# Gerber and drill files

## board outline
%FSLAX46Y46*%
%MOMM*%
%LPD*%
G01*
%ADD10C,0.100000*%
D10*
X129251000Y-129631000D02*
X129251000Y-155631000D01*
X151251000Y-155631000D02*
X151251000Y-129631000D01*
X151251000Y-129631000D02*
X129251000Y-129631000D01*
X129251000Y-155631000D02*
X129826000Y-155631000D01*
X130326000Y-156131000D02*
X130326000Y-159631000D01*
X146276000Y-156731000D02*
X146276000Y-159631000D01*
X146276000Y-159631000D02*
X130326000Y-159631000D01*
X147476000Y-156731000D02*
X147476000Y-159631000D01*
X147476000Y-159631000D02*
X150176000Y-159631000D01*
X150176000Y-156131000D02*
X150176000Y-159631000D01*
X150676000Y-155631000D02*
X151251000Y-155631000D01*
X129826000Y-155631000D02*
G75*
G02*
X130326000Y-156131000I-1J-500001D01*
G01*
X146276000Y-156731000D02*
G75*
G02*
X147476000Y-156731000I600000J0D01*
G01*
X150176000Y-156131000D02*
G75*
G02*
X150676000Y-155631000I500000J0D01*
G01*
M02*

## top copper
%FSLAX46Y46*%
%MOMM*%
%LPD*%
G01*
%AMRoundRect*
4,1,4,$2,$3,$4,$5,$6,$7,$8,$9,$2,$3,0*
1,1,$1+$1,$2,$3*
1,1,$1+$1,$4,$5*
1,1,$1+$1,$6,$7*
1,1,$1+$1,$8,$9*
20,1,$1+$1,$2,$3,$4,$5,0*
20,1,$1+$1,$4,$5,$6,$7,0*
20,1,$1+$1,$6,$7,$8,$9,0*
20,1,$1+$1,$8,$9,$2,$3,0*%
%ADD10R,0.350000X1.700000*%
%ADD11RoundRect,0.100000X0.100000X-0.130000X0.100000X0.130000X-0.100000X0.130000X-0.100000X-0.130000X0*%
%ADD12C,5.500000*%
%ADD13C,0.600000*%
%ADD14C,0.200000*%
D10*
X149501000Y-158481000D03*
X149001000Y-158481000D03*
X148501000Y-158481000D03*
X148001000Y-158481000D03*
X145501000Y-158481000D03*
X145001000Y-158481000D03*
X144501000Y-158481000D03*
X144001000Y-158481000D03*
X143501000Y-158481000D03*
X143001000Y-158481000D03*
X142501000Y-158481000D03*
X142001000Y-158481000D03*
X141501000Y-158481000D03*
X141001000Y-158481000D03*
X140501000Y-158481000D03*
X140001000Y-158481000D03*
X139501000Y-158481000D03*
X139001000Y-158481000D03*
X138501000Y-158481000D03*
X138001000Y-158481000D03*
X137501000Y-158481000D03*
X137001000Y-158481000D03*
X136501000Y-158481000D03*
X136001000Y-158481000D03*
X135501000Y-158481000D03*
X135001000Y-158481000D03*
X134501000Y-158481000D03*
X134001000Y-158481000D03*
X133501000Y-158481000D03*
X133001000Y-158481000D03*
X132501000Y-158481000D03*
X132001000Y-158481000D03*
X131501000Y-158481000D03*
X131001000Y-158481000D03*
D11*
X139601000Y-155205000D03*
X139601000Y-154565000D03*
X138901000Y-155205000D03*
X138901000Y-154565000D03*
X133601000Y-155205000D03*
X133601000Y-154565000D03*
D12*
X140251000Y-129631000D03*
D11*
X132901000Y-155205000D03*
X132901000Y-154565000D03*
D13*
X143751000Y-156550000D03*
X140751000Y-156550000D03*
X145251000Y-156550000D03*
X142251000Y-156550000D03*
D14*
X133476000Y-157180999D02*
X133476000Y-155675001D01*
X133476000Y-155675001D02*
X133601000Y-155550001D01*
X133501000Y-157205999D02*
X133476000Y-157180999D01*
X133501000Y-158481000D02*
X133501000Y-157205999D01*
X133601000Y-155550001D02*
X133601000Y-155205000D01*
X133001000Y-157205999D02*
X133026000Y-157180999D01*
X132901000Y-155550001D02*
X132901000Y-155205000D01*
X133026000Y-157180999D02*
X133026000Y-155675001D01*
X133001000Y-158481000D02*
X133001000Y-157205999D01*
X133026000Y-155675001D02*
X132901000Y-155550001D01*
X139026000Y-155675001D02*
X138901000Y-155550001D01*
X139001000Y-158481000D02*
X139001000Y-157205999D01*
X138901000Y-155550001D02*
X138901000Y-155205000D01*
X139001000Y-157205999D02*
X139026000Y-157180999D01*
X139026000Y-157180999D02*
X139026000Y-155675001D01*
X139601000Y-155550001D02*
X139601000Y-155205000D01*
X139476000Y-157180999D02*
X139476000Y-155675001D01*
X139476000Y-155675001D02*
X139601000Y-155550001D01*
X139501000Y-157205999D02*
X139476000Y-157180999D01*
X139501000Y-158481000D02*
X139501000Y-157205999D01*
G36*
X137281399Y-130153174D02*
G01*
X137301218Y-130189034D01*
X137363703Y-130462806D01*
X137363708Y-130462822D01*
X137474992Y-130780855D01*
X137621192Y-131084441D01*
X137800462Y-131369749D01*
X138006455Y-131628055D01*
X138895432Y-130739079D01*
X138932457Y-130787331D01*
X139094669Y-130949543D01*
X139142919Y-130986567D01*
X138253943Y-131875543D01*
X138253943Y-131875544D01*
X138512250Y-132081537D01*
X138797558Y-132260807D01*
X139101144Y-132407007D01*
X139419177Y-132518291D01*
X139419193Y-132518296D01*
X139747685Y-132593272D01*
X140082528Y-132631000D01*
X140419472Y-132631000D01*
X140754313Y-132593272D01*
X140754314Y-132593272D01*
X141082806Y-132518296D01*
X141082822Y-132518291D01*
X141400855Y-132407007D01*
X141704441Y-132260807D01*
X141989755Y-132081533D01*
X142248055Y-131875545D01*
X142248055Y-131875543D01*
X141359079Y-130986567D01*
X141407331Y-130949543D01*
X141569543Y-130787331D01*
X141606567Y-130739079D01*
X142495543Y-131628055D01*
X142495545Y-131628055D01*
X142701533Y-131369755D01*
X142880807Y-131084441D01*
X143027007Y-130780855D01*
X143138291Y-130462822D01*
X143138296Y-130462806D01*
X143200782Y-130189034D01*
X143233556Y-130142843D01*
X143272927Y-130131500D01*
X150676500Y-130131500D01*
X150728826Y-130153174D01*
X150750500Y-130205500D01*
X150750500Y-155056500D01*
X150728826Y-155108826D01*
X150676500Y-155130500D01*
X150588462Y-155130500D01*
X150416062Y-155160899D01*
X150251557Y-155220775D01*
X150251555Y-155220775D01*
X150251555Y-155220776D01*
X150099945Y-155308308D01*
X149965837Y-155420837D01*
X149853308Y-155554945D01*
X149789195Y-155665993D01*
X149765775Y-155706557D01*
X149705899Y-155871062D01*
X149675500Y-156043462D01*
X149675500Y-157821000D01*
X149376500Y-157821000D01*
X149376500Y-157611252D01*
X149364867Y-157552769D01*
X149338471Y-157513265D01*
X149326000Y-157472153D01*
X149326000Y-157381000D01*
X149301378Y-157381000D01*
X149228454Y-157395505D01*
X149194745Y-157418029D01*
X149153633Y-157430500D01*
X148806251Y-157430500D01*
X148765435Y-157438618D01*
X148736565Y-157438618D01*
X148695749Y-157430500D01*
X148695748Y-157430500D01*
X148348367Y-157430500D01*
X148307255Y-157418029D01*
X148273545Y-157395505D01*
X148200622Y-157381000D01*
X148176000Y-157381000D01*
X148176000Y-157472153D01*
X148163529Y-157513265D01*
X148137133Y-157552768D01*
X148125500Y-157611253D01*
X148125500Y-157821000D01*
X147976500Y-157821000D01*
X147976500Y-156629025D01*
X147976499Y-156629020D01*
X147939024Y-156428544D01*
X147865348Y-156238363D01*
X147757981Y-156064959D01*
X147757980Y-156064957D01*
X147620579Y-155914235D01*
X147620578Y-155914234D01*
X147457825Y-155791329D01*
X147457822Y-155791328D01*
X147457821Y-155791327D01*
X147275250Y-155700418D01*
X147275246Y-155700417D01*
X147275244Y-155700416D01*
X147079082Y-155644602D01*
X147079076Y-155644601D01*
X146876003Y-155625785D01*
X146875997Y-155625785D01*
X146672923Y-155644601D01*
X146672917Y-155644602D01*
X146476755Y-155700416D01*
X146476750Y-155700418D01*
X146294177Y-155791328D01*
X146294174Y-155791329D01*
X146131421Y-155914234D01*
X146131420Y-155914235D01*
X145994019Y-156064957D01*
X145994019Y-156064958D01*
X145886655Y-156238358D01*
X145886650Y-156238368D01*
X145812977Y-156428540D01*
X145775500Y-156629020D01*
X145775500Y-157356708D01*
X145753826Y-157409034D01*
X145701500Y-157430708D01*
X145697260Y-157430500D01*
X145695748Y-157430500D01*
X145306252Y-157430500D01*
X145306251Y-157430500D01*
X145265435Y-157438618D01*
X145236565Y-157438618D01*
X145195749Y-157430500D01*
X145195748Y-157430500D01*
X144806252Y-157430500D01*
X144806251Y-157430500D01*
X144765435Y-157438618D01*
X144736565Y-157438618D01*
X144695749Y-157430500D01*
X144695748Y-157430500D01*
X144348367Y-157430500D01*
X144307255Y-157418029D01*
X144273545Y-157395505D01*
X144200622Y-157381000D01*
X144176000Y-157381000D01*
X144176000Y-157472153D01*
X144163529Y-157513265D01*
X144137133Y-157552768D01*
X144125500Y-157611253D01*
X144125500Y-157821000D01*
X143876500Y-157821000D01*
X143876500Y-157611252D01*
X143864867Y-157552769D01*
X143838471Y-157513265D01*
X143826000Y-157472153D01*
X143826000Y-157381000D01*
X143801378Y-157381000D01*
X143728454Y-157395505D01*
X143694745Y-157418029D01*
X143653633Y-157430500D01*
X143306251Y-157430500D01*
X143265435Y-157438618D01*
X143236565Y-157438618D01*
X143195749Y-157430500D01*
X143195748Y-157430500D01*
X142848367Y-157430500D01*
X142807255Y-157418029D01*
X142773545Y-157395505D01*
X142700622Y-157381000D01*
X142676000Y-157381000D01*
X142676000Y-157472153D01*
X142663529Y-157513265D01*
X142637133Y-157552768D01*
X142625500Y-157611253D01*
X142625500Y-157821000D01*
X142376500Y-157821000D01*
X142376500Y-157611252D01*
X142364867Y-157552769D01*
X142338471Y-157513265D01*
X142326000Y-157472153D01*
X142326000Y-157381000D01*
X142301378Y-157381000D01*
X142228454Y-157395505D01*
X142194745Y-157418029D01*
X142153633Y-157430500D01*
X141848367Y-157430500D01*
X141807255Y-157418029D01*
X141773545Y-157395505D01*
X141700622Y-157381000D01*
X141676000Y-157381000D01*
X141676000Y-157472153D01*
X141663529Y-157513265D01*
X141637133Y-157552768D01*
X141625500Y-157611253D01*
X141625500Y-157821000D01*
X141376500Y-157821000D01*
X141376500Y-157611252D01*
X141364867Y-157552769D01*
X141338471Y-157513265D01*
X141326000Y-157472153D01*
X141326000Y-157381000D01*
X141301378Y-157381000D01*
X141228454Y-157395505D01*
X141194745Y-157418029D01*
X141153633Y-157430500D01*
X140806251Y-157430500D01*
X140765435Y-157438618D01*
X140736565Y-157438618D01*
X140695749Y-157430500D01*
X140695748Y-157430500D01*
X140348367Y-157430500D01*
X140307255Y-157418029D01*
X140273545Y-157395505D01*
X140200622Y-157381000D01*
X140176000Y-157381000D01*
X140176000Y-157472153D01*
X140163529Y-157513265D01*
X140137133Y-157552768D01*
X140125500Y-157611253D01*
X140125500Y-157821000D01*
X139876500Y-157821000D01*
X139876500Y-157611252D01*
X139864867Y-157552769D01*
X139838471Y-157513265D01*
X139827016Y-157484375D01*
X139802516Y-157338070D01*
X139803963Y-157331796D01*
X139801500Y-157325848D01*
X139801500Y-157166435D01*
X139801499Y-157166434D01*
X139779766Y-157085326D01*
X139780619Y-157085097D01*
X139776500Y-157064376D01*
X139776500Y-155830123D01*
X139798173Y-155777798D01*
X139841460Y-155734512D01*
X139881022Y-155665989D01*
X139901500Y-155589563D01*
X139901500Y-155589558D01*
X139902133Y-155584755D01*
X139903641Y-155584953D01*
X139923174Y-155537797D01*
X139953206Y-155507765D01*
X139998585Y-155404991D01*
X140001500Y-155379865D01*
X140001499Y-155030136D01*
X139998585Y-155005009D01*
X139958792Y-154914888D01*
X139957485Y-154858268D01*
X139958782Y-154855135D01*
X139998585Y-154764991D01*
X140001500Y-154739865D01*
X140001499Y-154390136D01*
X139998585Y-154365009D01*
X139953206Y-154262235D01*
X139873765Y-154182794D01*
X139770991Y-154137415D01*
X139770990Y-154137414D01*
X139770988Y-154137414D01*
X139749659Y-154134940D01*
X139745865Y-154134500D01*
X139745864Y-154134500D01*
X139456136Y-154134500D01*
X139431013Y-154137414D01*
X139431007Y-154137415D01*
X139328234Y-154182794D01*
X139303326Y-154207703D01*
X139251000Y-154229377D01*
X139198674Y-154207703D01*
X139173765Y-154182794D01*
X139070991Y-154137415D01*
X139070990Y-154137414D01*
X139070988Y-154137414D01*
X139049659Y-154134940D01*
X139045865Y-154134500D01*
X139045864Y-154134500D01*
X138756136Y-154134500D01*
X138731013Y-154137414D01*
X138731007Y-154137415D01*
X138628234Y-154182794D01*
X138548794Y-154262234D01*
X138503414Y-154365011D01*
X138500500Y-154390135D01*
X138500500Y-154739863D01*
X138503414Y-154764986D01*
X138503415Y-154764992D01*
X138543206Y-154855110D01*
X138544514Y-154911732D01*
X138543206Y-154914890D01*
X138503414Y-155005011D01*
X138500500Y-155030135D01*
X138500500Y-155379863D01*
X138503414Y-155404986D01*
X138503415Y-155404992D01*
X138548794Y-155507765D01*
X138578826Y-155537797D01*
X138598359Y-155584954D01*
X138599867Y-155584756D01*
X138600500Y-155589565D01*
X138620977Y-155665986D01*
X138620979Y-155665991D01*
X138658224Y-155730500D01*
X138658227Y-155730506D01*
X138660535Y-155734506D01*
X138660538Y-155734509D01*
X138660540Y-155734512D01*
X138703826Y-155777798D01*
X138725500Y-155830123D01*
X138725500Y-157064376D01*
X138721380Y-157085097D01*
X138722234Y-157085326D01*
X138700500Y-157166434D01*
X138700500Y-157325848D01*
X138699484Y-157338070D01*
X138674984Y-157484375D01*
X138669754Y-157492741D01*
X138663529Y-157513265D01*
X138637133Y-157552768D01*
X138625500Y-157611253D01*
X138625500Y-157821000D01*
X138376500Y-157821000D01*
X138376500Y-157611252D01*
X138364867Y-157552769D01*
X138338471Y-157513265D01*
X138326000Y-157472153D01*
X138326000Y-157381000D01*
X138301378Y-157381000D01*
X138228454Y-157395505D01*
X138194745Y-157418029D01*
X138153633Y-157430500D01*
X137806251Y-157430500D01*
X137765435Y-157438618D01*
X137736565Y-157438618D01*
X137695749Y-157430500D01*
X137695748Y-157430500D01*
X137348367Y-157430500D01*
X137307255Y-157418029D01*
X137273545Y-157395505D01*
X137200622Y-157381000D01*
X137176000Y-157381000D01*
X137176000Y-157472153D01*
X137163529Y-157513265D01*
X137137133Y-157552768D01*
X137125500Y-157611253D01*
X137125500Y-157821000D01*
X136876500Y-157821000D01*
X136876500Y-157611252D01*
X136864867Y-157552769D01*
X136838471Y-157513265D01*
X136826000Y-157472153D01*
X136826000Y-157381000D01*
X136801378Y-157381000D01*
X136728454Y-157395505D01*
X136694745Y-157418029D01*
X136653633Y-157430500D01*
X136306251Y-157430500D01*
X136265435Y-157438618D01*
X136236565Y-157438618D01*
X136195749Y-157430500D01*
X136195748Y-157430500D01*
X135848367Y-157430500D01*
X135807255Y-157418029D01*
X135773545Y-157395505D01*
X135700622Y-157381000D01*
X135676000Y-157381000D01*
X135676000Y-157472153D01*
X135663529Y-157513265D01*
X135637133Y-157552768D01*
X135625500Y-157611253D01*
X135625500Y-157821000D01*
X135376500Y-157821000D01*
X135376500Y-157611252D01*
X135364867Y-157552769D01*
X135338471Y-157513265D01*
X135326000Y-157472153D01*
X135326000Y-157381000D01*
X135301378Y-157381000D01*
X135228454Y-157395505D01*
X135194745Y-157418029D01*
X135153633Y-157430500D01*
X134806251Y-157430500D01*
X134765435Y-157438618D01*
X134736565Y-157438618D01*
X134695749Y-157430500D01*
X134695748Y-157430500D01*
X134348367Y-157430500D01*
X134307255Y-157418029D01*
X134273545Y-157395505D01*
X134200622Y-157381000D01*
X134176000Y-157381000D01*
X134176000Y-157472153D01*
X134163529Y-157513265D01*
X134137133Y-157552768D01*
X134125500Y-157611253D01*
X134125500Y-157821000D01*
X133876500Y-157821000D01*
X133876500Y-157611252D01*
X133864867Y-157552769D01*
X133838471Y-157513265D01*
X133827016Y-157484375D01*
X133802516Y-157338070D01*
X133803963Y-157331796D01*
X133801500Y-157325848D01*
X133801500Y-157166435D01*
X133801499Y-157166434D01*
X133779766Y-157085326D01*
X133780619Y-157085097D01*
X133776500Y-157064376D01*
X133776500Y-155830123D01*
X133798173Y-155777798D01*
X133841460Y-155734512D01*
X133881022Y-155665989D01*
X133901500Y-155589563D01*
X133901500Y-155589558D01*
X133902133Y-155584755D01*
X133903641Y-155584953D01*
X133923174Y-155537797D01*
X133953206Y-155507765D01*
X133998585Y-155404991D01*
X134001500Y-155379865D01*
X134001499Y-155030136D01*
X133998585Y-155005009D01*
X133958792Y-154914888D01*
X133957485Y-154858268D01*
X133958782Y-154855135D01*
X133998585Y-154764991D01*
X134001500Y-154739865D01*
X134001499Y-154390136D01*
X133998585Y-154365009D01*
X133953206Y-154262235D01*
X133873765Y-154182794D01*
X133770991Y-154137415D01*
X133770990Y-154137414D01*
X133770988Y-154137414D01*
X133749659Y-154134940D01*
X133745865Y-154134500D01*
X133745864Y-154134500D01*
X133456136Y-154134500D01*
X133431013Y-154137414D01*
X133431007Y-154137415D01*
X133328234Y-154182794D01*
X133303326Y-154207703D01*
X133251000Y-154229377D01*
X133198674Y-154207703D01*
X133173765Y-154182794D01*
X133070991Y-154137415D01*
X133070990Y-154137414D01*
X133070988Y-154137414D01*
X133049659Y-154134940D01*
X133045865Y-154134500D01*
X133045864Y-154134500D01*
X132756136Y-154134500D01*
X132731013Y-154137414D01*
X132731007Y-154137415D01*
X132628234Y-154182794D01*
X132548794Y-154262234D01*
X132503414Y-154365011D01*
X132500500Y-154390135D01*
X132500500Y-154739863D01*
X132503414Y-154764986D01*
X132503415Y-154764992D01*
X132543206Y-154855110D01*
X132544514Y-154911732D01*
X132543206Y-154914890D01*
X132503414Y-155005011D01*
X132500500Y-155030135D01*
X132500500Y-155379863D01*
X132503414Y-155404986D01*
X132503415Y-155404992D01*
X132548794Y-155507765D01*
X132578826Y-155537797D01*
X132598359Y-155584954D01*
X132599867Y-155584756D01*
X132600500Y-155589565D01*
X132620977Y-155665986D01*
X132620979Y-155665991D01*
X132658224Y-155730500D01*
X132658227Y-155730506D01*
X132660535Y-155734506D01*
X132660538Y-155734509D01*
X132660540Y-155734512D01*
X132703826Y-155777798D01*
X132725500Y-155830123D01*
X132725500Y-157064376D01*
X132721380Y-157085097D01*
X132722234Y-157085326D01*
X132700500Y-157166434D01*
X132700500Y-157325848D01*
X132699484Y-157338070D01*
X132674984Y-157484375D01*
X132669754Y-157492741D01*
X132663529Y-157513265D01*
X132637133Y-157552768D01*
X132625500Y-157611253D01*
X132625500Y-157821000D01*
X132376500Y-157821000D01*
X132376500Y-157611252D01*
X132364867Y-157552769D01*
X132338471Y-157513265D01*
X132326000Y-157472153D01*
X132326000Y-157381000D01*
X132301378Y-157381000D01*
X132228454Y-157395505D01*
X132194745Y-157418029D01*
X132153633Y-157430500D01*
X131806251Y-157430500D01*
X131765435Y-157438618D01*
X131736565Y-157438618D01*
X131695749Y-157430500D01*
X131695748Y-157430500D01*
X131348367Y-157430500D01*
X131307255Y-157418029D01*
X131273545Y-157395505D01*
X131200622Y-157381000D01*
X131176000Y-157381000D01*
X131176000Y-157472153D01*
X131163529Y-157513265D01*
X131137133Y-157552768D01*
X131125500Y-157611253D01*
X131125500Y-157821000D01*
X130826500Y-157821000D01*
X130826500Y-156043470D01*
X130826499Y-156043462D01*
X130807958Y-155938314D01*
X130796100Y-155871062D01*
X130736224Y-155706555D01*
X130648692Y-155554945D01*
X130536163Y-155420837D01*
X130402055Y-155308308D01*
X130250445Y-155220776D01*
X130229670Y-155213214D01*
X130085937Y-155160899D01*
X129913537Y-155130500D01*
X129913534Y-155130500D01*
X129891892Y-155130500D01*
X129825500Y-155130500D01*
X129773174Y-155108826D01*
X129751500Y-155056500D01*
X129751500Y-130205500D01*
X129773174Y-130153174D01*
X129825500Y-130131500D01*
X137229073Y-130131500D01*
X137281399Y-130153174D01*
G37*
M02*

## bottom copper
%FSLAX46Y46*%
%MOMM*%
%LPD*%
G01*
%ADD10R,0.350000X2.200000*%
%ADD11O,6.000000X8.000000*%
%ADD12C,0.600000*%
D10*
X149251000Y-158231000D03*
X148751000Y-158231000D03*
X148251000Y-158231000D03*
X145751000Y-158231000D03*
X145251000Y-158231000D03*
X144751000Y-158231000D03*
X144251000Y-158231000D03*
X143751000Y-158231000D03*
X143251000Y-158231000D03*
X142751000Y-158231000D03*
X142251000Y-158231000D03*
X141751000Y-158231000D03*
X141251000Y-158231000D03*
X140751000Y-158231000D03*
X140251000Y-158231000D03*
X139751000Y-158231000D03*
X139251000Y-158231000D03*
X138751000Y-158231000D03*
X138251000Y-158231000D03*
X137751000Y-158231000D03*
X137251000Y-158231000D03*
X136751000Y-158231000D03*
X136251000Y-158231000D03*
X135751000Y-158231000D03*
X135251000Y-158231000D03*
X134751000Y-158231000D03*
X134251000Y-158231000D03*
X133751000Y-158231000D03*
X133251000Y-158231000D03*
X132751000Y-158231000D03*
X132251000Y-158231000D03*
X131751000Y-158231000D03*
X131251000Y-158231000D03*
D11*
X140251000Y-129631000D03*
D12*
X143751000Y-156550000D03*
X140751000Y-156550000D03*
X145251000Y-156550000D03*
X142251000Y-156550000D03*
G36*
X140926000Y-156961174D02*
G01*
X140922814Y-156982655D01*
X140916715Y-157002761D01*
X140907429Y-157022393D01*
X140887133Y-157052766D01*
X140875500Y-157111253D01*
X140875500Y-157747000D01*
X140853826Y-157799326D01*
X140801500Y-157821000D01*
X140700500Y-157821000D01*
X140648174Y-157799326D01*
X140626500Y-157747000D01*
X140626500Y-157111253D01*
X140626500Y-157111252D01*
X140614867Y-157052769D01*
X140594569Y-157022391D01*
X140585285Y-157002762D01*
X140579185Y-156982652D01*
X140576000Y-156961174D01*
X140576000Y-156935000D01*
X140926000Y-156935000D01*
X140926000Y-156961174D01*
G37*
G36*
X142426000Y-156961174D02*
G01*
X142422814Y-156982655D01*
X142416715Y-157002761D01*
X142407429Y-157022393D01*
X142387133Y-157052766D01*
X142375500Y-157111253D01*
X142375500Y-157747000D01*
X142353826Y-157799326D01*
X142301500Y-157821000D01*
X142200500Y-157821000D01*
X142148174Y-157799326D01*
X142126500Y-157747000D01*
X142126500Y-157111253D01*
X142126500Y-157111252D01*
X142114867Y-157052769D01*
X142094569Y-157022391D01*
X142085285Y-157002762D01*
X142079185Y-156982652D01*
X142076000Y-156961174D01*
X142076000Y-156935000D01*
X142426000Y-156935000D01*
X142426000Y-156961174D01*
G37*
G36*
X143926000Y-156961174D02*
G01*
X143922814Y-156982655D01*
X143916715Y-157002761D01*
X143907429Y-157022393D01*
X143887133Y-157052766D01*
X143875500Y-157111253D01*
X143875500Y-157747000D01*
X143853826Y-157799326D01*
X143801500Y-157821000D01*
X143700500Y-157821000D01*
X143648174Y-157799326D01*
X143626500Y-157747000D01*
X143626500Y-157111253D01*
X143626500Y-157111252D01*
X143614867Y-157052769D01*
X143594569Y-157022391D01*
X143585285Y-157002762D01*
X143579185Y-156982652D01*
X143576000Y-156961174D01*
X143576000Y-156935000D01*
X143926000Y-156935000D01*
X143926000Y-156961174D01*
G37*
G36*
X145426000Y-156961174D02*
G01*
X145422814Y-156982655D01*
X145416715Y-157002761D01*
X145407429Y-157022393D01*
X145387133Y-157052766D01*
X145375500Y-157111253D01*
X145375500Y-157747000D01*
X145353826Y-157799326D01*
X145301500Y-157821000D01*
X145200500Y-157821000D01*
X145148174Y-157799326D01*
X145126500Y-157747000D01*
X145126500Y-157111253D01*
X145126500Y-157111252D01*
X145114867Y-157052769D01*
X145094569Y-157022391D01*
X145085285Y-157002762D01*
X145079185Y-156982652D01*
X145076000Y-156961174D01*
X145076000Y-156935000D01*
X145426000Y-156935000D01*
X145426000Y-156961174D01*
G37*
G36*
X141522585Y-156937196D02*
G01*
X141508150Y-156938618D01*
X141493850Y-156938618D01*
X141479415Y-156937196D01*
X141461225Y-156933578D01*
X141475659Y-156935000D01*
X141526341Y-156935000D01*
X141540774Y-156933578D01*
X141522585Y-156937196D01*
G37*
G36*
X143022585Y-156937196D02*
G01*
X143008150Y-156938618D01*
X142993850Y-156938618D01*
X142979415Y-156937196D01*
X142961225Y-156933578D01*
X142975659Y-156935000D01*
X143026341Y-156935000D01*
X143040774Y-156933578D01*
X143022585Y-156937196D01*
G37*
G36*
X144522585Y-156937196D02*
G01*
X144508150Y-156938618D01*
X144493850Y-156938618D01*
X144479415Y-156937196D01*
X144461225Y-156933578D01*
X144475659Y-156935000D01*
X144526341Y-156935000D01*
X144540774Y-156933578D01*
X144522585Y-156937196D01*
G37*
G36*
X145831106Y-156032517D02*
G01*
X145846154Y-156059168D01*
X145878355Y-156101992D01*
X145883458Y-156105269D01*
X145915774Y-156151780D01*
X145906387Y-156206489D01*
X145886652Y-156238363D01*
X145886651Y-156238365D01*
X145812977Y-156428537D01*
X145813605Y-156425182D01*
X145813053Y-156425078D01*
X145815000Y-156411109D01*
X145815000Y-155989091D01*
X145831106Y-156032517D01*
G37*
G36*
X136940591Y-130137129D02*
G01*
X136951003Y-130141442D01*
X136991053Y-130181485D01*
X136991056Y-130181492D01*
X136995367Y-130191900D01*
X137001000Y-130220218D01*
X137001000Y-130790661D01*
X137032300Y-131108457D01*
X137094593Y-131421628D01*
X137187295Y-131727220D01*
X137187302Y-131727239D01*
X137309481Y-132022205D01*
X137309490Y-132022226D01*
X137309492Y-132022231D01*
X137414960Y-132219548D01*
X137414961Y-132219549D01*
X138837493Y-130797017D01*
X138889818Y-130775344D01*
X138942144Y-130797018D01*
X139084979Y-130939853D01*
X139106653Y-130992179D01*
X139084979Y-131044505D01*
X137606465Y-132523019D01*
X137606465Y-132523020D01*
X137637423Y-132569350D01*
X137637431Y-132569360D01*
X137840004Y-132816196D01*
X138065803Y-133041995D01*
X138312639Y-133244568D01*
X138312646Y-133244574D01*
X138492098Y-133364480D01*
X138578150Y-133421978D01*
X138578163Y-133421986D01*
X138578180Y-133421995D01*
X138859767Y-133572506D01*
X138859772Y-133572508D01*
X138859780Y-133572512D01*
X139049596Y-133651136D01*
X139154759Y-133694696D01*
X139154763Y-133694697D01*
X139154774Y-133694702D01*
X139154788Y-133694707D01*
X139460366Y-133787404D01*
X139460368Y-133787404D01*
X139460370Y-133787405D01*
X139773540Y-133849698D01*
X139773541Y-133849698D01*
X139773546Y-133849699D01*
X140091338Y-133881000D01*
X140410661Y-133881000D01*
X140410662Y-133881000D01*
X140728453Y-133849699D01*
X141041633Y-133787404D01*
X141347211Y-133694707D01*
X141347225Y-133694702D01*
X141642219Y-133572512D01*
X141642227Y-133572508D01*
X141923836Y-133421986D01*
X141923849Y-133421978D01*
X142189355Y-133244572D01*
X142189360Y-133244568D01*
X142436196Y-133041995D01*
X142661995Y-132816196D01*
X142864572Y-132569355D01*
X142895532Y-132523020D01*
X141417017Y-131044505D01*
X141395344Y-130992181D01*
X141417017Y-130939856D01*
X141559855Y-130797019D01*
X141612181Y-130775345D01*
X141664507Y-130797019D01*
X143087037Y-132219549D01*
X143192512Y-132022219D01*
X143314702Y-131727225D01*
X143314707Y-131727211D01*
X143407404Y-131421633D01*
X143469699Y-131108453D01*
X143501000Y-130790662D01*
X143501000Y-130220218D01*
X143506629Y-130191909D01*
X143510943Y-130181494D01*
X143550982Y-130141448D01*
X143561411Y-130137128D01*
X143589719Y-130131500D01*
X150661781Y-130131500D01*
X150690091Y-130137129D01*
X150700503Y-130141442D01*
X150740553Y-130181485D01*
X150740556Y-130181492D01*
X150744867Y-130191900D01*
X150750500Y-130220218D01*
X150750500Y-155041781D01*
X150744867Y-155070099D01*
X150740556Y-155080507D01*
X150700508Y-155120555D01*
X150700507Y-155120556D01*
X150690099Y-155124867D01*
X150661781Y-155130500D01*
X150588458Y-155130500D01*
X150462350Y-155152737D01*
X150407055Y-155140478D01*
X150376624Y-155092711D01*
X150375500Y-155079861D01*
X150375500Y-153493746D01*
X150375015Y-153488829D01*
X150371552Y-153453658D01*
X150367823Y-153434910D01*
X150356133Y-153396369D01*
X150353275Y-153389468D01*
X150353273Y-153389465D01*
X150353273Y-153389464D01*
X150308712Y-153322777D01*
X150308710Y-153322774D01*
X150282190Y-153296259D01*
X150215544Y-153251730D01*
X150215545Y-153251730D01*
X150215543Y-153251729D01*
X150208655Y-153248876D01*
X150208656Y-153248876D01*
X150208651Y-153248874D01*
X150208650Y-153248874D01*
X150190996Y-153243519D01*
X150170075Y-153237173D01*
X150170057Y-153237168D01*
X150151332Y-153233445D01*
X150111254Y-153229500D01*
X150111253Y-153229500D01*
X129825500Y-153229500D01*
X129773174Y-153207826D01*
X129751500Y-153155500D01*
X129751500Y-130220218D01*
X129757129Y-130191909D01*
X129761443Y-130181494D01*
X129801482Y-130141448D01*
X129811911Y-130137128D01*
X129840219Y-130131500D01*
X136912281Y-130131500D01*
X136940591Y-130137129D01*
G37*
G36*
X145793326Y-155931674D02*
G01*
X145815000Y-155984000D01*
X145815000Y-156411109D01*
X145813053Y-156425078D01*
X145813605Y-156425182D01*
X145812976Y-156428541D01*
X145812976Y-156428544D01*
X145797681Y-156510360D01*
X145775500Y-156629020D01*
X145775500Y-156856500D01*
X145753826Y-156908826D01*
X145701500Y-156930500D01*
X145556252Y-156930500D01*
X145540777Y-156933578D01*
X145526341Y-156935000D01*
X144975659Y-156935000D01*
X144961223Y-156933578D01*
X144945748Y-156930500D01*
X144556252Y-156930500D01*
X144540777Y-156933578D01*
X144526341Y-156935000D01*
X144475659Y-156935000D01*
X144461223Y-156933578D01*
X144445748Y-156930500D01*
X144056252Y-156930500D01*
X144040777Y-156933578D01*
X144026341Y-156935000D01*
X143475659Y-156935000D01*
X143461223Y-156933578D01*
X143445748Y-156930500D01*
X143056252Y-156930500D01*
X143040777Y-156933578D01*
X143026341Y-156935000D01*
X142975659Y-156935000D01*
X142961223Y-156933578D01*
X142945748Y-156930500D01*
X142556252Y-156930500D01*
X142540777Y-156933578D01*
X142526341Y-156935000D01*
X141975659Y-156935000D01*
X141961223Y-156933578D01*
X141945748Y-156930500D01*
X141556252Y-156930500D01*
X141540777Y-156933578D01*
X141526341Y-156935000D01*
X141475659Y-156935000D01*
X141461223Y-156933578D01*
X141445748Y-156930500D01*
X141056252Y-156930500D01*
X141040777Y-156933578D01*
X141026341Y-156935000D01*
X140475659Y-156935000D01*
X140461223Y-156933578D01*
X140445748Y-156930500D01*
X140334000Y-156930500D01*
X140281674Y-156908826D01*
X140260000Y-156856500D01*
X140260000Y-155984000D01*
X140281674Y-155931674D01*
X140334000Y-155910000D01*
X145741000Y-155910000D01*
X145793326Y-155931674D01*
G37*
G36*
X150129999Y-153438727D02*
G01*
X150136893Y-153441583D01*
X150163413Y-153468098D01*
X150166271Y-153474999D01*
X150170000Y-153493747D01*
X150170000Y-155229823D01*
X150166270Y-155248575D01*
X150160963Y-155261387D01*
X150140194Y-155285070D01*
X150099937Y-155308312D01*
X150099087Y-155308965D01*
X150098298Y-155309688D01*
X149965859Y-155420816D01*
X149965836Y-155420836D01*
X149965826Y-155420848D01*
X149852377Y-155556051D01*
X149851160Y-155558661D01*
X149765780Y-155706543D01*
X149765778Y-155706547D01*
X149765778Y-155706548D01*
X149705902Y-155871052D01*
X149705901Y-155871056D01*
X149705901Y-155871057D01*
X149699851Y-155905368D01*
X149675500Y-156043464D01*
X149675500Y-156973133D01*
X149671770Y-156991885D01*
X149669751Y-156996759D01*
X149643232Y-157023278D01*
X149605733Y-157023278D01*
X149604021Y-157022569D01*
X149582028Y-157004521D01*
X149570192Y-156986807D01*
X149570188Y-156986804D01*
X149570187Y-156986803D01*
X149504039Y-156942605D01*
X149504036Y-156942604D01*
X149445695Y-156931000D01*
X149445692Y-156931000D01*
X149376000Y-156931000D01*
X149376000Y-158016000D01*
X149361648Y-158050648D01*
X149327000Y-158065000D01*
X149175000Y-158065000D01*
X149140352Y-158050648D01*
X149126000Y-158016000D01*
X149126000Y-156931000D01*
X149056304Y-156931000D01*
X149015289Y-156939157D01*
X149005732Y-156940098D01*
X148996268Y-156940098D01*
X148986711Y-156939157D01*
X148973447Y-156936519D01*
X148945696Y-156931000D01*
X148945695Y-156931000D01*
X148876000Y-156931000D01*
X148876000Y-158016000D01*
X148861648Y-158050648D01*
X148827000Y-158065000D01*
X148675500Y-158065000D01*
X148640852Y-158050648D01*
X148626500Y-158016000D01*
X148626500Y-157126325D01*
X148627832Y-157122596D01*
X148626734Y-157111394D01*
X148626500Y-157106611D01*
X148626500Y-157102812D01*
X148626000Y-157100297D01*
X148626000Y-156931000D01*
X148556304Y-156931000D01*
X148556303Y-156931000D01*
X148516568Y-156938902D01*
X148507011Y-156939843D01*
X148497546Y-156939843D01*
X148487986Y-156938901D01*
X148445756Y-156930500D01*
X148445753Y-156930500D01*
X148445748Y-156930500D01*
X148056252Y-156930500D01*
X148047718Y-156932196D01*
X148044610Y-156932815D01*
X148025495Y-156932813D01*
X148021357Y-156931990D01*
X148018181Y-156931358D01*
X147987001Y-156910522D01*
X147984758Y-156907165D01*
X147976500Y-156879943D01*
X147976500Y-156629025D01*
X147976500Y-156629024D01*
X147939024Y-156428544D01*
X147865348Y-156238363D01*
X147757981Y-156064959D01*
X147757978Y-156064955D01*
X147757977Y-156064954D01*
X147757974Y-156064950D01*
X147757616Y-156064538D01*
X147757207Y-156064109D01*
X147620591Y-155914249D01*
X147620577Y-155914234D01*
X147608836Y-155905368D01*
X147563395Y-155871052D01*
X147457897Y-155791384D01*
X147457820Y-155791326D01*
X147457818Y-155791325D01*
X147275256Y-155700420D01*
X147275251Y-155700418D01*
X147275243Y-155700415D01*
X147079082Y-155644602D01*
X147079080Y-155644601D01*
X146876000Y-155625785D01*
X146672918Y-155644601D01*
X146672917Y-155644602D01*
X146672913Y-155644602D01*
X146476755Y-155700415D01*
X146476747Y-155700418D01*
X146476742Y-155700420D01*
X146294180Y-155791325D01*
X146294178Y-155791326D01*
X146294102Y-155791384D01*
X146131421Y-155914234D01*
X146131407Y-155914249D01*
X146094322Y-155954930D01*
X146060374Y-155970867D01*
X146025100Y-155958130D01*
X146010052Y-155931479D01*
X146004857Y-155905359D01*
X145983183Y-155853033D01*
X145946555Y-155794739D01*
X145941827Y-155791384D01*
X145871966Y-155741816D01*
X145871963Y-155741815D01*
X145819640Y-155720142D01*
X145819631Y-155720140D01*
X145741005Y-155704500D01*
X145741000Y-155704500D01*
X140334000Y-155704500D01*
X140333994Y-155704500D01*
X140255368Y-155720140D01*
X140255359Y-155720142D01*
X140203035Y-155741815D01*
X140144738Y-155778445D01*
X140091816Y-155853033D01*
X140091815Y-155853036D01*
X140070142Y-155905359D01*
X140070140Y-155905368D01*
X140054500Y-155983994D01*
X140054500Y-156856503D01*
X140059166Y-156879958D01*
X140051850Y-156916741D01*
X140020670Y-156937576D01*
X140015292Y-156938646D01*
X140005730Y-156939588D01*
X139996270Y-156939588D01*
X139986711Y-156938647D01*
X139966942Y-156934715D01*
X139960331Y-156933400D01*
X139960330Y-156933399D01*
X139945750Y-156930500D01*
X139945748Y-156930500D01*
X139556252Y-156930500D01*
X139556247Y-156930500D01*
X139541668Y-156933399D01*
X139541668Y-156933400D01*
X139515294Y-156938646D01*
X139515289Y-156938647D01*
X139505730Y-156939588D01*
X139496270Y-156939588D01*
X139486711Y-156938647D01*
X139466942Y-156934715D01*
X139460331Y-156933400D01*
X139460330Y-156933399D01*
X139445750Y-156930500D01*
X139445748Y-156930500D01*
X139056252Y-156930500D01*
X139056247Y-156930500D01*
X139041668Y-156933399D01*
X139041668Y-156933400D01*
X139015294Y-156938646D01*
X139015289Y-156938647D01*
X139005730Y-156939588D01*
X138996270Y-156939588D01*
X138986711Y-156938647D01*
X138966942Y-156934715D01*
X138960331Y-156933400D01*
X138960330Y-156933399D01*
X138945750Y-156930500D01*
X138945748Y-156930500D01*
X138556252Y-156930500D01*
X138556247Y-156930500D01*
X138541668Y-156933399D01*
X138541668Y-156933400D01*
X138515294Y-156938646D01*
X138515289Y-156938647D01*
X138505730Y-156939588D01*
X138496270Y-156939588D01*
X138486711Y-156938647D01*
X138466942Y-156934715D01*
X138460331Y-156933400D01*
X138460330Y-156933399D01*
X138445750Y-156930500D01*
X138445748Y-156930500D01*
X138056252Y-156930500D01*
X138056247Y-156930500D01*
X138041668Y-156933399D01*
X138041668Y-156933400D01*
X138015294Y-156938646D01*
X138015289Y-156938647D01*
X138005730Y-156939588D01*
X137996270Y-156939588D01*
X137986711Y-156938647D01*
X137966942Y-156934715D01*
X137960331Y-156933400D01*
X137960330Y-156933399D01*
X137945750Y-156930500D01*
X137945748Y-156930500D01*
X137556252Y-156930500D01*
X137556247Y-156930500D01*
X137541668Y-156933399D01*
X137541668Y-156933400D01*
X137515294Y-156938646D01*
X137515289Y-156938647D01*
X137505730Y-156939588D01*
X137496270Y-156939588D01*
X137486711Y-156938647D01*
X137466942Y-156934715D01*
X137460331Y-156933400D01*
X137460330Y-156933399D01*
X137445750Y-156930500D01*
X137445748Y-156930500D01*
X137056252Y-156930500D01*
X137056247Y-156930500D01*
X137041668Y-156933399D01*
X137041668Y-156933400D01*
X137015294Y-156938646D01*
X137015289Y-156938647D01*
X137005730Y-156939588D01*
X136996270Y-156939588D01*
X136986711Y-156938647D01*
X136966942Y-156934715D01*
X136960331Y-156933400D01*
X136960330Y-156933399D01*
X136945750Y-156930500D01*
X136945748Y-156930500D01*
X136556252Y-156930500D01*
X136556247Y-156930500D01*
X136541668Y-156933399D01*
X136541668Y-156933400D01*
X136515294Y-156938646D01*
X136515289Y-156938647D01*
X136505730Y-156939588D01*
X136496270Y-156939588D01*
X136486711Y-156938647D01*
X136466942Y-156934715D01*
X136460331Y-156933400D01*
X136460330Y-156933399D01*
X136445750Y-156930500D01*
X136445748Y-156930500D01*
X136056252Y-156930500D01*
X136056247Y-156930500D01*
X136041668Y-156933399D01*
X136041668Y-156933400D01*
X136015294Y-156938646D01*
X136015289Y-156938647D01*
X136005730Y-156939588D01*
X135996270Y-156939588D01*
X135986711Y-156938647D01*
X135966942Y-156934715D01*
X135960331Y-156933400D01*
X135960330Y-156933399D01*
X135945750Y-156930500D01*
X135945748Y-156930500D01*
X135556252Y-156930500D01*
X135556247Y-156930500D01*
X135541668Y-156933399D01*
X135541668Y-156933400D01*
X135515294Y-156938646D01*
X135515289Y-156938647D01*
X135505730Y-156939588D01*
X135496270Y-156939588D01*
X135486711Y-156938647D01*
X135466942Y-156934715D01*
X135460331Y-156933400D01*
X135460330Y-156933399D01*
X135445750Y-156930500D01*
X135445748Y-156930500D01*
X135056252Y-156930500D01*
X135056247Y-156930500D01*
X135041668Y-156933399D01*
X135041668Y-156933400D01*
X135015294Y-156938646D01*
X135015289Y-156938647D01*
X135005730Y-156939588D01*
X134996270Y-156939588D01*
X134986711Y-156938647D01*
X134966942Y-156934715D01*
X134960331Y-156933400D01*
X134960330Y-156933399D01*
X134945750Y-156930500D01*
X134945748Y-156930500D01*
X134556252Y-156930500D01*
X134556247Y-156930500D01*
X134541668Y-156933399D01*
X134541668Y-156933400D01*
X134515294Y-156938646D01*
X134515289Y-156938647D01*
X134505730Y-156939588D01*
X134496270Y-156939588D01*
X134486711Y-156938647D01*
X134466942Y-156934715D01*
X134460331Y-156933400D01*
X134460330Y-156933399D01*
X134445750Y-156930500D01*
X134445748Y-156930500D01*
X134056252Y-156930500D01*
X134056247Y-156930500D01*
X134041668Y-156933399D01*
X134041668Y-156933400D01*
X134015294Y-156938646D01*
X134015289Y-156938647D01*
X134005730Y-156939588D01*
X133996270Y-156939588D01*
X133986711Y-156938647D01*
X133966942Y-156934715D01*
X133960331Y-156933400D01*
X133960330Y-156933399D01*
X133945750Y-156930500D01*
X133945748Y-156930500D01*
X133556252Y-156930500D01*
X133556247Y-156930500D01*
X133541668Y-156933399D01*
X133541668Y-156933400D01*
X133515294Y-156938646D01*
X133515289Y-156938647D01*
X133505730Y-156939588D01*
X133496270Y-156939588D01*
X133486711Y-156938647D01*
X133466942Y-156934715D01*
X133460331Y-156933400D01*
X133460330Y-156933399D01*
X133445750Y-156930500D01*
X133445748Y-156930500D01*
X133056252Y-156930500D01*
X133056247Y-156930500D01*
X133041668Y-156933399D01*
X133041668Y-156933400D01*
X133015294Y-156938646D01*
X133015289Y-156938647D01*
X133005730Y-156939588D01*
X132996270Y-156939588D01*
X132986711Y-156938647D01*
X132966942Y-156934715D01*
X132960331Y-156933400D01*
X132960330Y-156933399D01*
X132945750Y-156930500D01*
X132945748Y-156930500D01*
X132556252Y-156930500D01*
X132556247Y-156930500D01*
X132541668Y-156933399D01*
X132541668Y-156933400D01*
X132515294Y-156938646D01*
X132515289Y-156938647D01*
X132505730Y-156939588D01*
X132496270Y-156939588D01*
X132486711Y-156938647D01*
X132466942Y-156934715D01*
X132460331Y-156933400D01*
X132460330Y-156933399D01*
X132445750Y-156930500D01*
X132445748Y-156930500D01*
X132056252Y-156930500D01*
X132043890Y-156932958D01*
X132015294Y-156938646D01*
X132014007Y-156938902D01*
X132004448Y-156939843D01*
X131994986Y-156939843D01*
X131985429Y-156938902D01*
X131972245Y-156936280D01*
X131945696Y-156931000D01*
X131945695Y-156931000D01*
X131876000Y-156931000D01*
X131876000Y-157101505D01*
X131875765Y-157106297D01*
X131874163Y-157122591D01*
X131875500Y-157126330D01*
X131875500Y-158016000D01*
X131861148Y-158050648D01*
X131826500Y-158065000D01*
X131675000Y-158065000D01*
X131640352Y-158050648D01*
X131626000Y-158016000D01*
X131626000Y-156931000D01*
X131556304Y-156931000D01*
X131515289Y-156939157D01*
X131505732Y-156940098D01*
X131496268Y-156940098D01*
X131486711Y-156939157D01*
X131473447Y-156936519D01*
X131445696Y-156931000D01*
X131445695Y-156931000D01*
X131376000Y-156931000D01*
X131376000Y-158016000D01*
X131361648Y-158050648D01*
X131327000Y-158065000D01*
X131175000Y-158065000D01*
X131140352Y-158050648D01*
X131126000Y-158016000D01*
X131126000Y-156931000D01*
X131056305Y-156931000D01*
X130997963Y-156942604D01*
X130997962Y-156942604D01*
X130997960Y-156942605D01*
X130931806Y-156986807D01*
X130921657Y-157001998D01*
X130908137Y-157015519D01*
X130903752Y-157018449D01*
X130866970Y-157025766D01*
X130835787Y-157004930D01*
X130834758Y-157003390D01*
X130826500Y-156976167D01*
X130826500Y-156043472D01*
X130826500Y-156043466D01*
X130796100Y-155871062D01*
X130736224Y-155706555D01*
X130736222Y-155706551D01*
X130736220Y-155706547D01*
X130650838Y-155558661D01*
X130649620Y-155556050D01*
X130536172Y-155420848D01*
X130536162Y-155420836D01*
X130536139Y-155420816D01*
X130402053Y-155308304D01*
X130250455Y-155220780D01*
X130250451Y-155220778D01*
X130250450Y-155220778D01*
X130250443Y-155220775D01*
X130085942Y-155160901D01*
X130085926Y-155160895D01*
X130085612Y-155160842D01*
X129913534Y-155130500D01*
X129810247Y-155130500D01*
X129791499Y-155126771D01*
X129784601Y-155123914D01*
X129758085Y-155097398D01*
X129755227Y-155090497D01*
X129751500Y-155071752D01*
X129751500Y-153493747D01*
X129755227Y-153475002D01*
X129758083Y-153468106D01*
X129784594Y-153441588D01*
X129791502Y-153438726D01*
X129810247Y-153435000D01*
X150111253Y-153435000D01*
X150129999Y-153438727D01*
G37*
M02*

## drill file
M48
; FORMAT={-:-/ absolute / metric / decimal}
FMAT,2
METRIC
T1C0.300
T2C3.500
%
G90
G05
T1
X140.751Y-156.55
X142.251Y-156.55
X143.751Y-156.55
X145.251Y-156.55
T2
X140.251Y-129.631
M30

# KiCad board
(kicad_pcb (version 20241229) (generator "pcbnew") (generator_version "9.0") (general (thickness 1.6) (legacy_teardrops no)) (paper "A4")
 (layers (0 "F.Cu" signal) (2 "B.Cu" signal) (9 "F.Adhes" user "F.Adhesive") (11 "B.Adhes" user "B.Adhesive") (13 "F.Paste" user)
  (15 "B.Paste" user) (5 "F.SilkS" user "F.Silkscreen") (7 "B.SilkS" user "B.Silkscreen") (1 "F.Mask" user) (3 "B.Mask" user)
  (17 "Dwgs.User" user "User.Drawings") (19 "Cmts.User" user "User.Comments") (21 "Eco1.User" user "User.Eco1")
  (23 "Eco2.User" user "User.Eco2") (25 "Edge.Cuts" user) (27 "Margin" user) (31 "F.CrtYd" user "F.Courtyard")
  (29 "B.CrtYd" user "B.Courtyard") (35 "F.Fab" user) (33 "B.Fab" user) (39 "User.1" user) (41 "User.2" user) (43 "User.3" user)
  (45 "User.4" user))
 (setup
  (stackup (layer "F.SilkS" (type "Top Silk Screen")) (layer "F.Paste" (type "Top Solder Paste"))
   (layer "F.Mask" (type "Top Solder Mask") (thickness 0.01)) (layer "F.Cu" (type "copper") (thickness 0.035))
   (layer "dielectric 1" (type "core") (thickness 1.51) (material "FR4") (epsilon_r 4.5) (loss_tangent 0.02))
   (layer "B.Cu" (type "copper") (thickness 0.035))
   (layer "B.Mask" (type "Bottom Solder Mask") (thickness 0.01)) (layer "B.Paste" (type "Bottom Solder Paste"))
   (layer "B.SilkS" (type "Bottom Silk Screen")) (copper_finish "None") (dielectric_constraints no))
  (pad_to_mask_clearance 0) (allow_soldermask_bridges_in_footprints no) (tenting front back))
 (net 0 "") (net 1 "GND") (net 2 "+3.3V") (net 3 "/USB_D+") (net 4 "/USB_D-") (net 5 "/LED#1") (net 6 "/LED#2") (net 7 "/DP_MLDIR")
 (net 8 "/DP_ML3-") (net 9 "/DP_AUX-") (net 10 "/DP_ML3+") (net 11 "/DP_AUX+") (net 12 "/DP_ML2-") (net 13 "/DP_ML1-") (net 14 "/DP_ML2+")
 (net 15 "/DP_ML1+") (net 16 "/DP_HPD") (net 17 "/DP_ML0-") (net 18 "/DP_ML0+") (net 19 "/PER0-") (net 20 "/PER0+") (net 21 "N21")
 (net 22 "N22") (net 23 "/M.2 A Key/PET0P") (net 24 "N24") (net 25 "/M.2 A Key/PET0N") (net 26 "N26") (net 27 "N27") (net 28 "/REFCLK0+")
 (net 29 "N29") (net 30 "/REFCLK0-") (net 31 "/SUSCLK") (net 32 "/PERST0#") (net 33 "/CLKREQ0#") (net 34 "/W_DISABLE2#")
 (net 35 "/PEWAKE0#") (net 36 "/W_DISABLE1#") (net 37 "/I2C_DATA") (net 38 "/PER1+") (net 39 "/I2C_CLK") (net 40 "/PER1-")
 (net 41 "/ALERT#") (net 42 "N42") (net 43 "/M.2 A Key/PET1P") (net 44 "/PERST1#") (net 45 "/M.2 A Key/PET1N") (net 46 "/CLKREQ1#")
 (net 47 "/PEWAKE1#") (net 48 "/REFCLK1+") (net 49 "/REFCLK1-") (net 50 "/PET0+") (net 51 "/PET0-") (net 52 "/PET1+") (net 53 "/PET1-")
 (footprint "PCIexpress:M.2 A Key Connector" (layer "F.Cu") (at 140.251 158.521)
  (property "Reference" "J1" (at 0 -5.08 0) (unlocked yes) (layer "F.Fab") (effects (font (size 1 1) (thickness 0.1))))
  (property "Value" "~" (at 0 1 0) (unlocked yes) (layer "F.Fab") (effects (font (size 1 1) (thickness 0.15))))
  (fp_line (start -11 -2.89) (end -10.425 -2.89) (stroke (width 0.1) (type default)) (layer "Edge.Cuts"))
  (fp_line (start -9.925 -2.39) (end -9.925 1.11) (stroke (width 0.1) (type default)) (layer "Edge.Cuts"))
  (fp_line (start 6.025 -1.79) (end 6.025 1.11) (stroke (width 0.1) (type default)) (layer "Edge.Cuts"))
  (fp_line (start 6.025 1.11) (end -9.925 1.11) (stroke (width 0.1) (type default)) (layer "Edge.Cuts"))
  (fp_line (start 7.225 -1.79) (end 7.225 1.11) (stroke (width 0.1) (type default)) (layer "Edge.Cuts"))
  (fp_line (start 7.225 1.11) (end 9.925 1.11) (stroke (width 0.1) (type default)) (layer "Edge.Cuts"))
  (fp_line (start 9.925 -2.39) (end 9.925 1.11) (stroke (width 0.1) (type default)) (layer "Edge.Cuts"))
  (fp_line (start 10.425 -2.89) (end 11 -2.89) (stroke (width 0.1) (type default)) (layer "Edge.Cuts"))
  (fp_arc (start -10.425 -2.89) (mid -10.071447 -2.743553) (end -9.925 -2.39) (stroke (width 0.1) (type default)) (layer "Edge.Cuts"))
  (fp_arc (start 6.025 -1.79) (mid 6.625 -2.39) (end 7.225 -1.79) (stroke (width 0.1) (type default)) (layer "Edge.Cuts"))
  (fp_arc (start 9.925 -2.39) (mid 10.071447 -2.743553) (end 10.425 -2.89) (stroke (width 0.1) (type default)) (layer "Edge.Cuts"))
  (pad "1" smd rect (at 9.25 -0.04 180) (size 0.35 1.7) (layers "F.Cu") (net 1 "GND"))
  (pad "2" smd rect (at 9 -0.29 180) (size 0.35 2.2) (layers "B.Cu") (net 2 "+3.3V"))
  (pad "3" smd rect (at 8.75 -0.04 180) (size 0.35 1.7) (layers "F.Cu") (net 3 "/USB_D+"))
  (pad "4" smd rect (at 8.5 -0.29 180) (size 0.35 2.2) (layers "B.Cu") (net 2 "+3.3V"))
  (pad "5" smd rect (at 8.25 -0.04 180) (size 0.35 1.7) (layers "F.Cu") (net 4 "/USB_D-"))
  (pad "6" smd rect (at 8 -0.29 180) (size 0.35 2.2) (layers "B.Cu") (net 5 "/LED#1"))
  (pad "7" smd rect (at 7.75 -0.04 180) (size 0.35 1.7) (layers "F.Cu") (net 1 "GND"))
  (pad "16" smd rect (at 5.5 -0.29 180) (size 0.35 2.2) (layers "B.Cu") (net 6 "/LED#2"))
  (pad "17" smd rect (at 5.25 -0.04 180) (size 0.35 1.7) (layers "F.Cu") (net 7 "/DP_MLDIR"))
  (pad "18" smd rect (at 5 -0.29 180) (size 0.35 2.2) (layers "B.Cu") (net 1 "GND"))
  (pad "19" smd rect (at 4.75 -0.04 180) (size 0.35 1.7) (layers "F.Cu") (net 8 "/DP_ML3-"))
  (pad "20" smd rect (at 4.5 -0.29 180) (size 0.35 2.2) (layers "B.Cu") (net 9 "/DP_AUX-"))
  (pad "21" smd rect (at 4.25 -0.04 180) (size 0.35 1.7) (layers "F.Cu") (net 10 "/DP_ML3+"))
  (pad "22" smd rect (at 4 -0.29 180) (size 0.35 2.2) (layers "B.Cu") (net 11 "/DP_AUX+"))
  (pad "23" smd rect (at 3.75 -0.04 180) (size 0.35 1.7) (layers "F.Cu") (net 1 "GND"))
  (pad "24" smd rect (at 3.5 -0.29 180) (size 0.35 2.2) (layers "B.Cu") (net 1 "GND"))
  (pad "25" smd rect (at 3.25 -0.04 180) (size 0.35 1.7) (layers "F.Cu") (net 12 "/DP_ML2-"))
  (pad "26" smd rect (at 3 -0.29 180) (size 0.35 2.2) (layers "B.Cu") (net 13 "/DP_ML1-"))
  (pad "27" smd rect (at 2.75 -0.04 180) (size 0.35 1.7) (layers "F.Cu") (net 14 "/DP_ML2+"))
  (pad "28" smd rect (at 2.5 -0.29 180) (size 0.35 2.2) (layers "B.Cu") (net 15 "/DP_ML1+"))
  (pad "29" smd rect (at 2.25 -0.04 180) (size 0.35 1.7) (layers "F.Cu") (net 1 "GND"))
  (pad "30" smd rect (at 2 -0.29 180) (size 0.35 2.2) (layers "B.Cu") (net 1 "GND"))
  (pad "31" smd rect (at 1.75 -0.04 180) (size 0.35 1.7) (layers "F.Cu") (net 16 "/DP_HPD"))
  (pad "32" smd rect (at 1.5 -0.29 180) (size 0.35 2.2) (layers "B.Cu") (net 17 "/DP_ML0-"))
  (pad "33" smd rect (at 1.25 -0.04 180) (size 0.35 1.7) (layers "F.Cu") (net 1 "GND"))
  (pad "34" smd rect (at 1 -0.29 180) (size 0.35 2.2) (layers "B.Cu") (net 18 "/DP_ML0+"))
  (pad "35" smd rect (at 0.75 -0.04 180) (size 0.35 1.7) (layers "F.Cu") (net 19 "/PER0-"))
  (pad "36" smd rect (at 0.5 -0.29 180) (size 0.35 2.2) (layers "B.Cu") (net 1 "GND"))
  (pad "37" smd rect (at 0.25 -0.04 180) (size 0.35 1.7) (layers "F.Cu") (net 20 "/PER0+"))
  (pad "38" smd rect (at 0 -0.29 180) (size 0.35 2.2) (layers "B.Cu") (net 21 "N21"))
  (pad "39" smd rect (at -0.25 -0.04 180) (size 0.35 1.7) (layers "F.Cu") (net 1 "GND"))
  (pad "40" smd rect (at -0.5 -0.29 180) (size 0.35 2.2) (layers "B.Cu") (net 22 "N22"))
  (pad "41" smd rect (at -0.75 -0.04 180) (size 0.35 1.7) (layers "F.Cu") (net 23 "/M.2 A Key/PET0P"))
  (pad "42" smd rect (at -1 -0.29 180) (size 0.35 2.2) (layers "B.Cu") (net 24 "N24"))
  (pad "43" smd rect (at -1.25 -0.04 180) (size 0.35 1.7) (layers "F.Cu") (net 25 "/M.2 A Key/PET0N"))
  (pad "44" smd rect (at -1.5 -0.29 180) (size 0.35 2.2) (layers "B.Cu") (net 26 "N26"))
  (pad "45" smd rect (at -1.75 -0.04 180) (size 0.35 1.7) (layers "F.Cu") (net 1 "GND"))
  (pad "46" smd rect (at -2 -0.29 180) (size 0.35 2.2) (layers "B.Cu") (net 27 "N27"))
  (pad "47" smd rect (at -2.25 -0.04 180) (size 0.35 1.7) (layers "F.Cu") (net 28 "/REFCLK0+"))
  (pad "48" smd rect (at -2.5 -0.29 180) (size 0.35 2.2) (layers "B.Cu") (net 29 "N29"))
  (pad "49" smd rect (at -2.75 -0.04 180) (size 0.35 1.7) (layers "F.Cu") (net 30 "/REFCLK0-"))
  (pad "50" smd rect (at -3 -0.29 180) (size 0.35 2.2) (layers "B.Cu") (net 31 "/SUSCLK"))
  (pad "51" smd rect (at -3.25 -0.04 180) (size 0.35 1.7) (layers "F.Cu") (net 1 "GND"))
  (pad "52" smd rect (at -3.5 -0.29 180) (size 0.35 2.2) (layers "B.Cu") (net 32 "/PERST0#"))
  (pad "53" smd rect (at -3.75 -0.04 180) (size 0.35 1.7) (layers "F.Cu") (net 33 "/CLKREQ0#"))
  (pad "54" smd rect (at -4 -0.29 180) (size 0.35 2.2) (layers "B.Cu") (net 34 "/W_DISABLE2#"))
  (pad "55" smd rect (at -4.25 -0.04 180) (size 0.35 1.7) (layers "F.Cu") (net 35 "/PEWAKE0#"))
  (pad "56" smd rect (at -4.5 -0.29 180) (size 0.35 2.2) (layers "B.Cu") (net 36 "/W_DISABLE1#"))
  (pad "57" smd rect (at -4.75 -0.04 180) (size 0.35 1.7) (layers "F.Cu") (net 1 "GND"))
  (pad "58" smd rect (at -5 -0.29 180) (size 0.35 2.2) (layers "B.Cu") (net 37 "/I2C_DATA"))
  (pad "59" smd rect (at -5.25 -0.04 180) (size 0.35 1.7) (layers "F.Cu") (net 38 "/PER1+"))
  (pad "60" smd rect (at -5.5 -0.29 180) (size 0.35 2.2) (layers "B.Cu") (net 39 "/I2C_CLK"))
  (pad "61" smd rect (at -5.75 -0.04 180) (size 0.35 1.7) (layers "F.Cu") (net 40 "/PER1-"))
  (pad "62" smd rect (at -6 -0.29 180) (size 0.35 2.2) (layers "B.Cu") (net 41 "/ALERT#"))
  (pad "63" smd rect (at -6.25 -0.04 180) (size 0.35 1.7) (layers "F.Cu") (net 1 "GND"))
  (pad "64" smd rect (at -6.5 -0.29 180) (size 0.35 2.2) (layers "B.Cu") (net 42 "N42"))
  (pad "65" smd rect (at -6.75 -0.04 180) (size 0.35 1.7) (layers "F.Cu") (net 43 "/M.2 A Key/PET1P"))
  (pad "66" smd rect (at -7 -0.29 180) (size 0.35 2.2) (layers "B.Cu") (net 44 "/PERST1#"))
  (pad "67" smd rect (at -7.25 -0.04 180) (size 0.35 1.7) (layers "F.Cu") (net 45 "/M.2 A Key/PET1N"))
  (pad "68" smd rect (at -7.5 -0.29 180) (size 0.35 2.2) (layers "B.Cu") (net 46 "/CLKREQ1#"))
  (pad "69" smd rect (at -7.75 -0.04 180) (size 0.35 1.7) (layers "F.Cu") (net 1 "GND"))
  (pad "70" smd rect (at -8 -0.29 180) (size 0.35 2.2) (layers "B.Cu") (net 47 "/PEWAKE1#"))
  (pad "71" smd rect (at -8.25 -0.04 180) (size 0.35 1.7) (layers "F.Cu") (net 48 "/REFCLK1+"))
  (pad "72" smd rect (at -8.5 -0.29 180) (size 0.35 2.2) (layers "B.Cu") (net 2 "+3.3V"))
  (pad "73" smd rect (at -8.75 -0.04 180) (size 0.35 1.7) (layers "F.Cu") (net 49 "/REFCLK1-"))
  (pad "74" smd rect (at -9 -0.29 180) (size 0.35 2.2) (layers "B.Cu") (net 2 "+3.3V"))
  (pad "75" smd rect (at -9.25 -0.04 180) (size 0.35 1.7) (layers "F.Cu") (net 1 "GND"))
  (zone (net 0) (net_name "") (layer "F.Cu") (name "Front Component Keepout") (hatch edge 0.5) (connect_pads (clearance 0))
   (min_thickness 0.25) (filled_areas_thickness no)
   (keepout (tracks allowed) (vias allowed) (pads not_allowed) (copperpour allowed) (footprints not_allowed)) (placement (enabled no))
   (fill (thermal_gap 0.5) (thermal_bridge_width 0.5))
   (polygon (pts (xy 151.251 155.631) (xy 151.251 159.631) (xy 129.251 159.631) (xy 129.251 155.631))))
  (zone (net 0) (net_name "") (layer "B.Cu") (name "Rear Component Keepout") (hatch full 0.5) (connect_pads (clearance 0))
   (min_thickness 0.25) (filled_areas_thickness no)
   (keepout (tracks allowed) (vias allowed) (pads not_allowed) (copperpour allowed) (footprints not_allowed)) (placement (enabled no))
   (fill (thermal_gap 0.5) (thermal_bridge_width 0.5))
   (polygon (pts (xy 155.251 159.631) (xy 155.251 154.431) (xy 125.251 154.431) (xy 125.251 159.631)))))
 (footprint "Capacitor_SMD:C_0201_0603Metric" (layer "F.Cu") (at 139.601 154.885 90)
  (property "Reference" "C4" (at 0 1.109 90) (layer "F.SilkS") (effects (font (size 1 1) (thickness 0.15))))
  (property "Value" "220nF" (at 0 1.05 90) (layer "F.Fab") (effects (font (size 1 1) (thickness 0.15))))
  (pad "" smd roundrect (at -0.345 0 90) (size 0.318 0.36) (layers "F.Paste") (roundrect_rratio 0.25))
  (pad "" smd roundrect (at 0.345 0 90) (size 0.318 0.36) (layers "F.Paste") (roundrect_rratio 0.25))
  (pad "1" smd roundrect (at -0.32 0 90) (size 0.46 0.4) (layers "F.Cu" "F.Mask") (roundrect_rratio 0.25) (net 23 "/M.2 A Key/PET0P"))
  (pad "2" smd roundrect (at 0.32 0 90) (size 0.46 0.4) (layers "F.Cu" "F.Mask") (roundrect_rratio 0.25) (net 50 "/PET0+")))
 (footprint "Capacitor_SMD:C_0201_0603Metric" (layer "F.Cu") (at 138.901 154.885 90)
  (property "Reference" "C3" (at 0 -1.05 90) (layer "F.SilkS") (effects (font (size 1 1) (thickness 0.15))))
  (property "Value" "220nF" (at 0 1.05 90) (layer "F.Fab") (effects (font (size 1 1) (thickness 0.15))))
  (pad "" smd roundrect (at -0.345 0 90) (size 0.318 0.36) (layers "F.Paste") (roundrect_rratio 0.25))
  (pad "" smd roundrect (at 0.345 0 90) (size 0.318 0.36) (layers "F.Paste") (roundrect_rratio 0.25))
  (pad "1" smd roundrect (at -0.32 0 90) (size 0.46 0.4) (layers "F.Cu" "F.Mask") (roundrect_rratio 0.25) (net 25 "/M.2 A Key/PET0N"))
  (pad "2" smd roundrect (at 0.32 0 90) (size 0.46 0.4) (layers "F.Cu" "F.Mask") (roundrect_rratio 0.25) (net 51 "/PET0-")))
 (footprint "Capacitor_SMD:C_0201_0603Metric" (layer "F.Cu") (at 133.601 154.885 90)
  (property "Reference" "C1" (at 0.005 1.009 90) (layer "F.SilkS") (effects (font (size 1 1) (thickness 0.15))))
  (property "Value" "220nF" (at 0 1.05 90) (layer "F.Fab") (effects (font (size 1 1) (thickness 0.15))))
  (pad "" smd roundrect (at -0.345 0 90) (size 0.318 0.36) (layers "F.Paste") (roundrect_rratio 0.25))
  (pad "" smd roundrect (at 0.345 0 90) (size 0.318 0.36) (layers "F.Paste") (roundrect_rratio 0.25))
  (pad "1" smd roundrect (at -0.32 0 90) (size 0.46 0.4) (layers "F.Cu" "F.Mask") (roundrect_rratio 0.25) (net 43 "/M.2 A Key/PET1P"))
  (pad "2" smd roundrect (at 0.32 0 90) (size 0.46 0.4) (layers "F.Cu" "F.Mask") (roundrect_rratio 0.25) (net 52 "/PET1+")))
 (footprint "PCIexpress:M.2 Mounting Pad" (layer "F.Cu") (at 140.251 129.631)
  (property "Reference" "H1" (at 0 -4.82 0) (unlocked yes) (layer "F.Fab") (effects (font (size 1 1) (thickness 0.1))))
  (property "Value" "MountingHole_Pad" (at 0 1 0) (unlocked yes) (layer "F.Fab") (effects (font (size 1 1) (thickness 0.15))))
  (pad "1" thru_hole circle (at 0 0) (size 5.5 5.5) (drill 3.5) (layers "*.Cu" "*.Mask") (remove_unused_layers no) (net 1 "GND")
   (padstack (mode front_inner_back)
    (layer "Inner" (shape circle) (size 5.5 5.5) (zone_connect -1))
    (layer "B.Cu" (shape oval) (size 6 8) (thermal_bridge_angle 45) (zone_connect -1)))))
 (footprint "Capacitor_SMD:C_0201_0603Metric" (layer "F.Cu") (at 132.901 154.885 90)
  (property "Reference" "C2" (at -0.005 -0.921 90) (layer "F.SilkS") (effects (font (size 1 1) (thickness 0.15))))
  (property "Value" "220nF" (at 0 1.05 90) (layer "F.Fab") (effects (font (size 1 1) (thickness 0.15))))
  (pad "" smd roundrect (at -0.345 0 90) (size 0.318 0.36) (layers "F.Paste") (roundrect_rratio 0.25))
  (pad "" smd roundrect (at 0.345 0 90) (size 0.318 0.36) (layers "F.Paste") (roundrect_rratio 0.25))
  (pad "1" smd roundrect (at -0.32 0 90) (size 0.46 0.4) (layers "F.Cu" "F.Mask") (roundrect_rratio 0.25) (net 45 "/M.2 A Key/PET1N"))
  (pad "2" smd roundrect (at 0.32 0 90) (size 0.46 0.4) (layers "F.Cu" "F.Mask") (roundrect_rratio 0.25) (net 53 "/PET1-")))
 (gr_line (start 129.251 129.631) (end 129.251 155.631) (stroke (width 0.1) (type default)) (layer "Edge.Cuts"))
 (gr_line (start 151.251 155.631) (end 151.251 129.631) (stroke (width 0.1) (type default)) (layer "Edge.Cuts"))
 (gr_line (start 151.251 129.631) (end 129.251 129.631) (stroke (width 0.1) (type solid)) (layer "Edge.Cuts"))
 (segment (start 133.476 157.180999) (end 133.476 155.675001) (width 0.2) (layer "F.Cu") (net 43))
 (segment (start 133.476 155.675001) (end 133.601 155.550001) (width 0.2) (layer "F.Cu") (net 43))
 (segment (start 133.501 157.205999) (end 133.476 157.180999) (width 0.2) (layer "F.Cu") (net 43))
 (segment (start 133.501 158.481) (end 133.501 157.205999) (width 0.2) (layer "F.Cu") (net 43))
 (segment (start 133.601 155.550001) (end 133.601 155.205) (width 0.2) (layer "F.Cu") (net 43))
 (segment (start 133.001 157.205999) (end 133.026 157.180999) (width 0.2) (layer "F.Cu") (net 45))
 (segment (start 132.901 155.550001) (end 132.901 155.205) (width 0.2) (layer "F.Cu") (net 45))
 (segment (start 133.026 157.180999) (end 133.026 155.675001) (width 0.2) (layer "F.Cu") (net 45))
 (segment (start 133.001 158.481) (end 133.001 157.205999) (width 0.2) (layer "F.Cu") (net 45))
 (segment (start 133.026 155.675001) (end 132.901 155.550001) (width 0.2) (layer "F.Cu") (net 45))
 (segment (start 139.026 155.675001) (end 138.901 155.550001) (width 0.2) (layer "F.Cu") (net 25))
 (segment (start 139.001 158.481) (end 139.001 157.205999) (width 0.2) (layer "F.Cu") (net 25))
 (segment (start 138.901 155.550001) (end 138.901 155.205) (width 0.2) (layer "F.Cu") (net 25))
 (segment (start 139.001 157.205999) (end 139.026 157.180999) (width 0.2) (layer "F.Cu") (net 25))
 (segment (start 139.026 157.180999) (end 139.026 155.675001) (width 0.2) (layer "F.Cu") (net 25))
 (segment (start 139.601 155.550001) (end 139.601 155.205) (width 0.2) (layer "F.Cu") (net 23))
 (segment (start 139.476 157.180999) (end 139.476 155.675001) (width 0.2) (layer "F.Cu") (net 23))
 (segment (start 139.476 155.675001) (end 139.601 155.550001) (width 0.2) (layer "F.Cu") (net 23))
 (segment (start 139.501 157.205999) (end 139.476 157.180999) (width 0.2) (layer "F.Cu") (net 23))
 (segment (start 139.501 158.481) (end 139.501 157.205999) (width 0.2) (layer "F.Cu") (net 23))
 (via (at 143.751 156.55) (size 0.6) (drill 0.3) (layers "F.Cu" "B.Cu") (free yes) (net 1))
 (via (at 140.751 156.55) (size 0.6) (drill 0.3) (layers "F.Cu" "B.Cu") (free yes) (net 1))
 (via (at 145.251 156.55) (size 0.6) (drill 0.3) (layers "F.Cu" "B.Cu") (free yes) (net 1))
 (via (at 142.251 156.55) (size 0.6) (drill 0.3) (layers "F.Cu" "B.Cu") (free yes) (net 1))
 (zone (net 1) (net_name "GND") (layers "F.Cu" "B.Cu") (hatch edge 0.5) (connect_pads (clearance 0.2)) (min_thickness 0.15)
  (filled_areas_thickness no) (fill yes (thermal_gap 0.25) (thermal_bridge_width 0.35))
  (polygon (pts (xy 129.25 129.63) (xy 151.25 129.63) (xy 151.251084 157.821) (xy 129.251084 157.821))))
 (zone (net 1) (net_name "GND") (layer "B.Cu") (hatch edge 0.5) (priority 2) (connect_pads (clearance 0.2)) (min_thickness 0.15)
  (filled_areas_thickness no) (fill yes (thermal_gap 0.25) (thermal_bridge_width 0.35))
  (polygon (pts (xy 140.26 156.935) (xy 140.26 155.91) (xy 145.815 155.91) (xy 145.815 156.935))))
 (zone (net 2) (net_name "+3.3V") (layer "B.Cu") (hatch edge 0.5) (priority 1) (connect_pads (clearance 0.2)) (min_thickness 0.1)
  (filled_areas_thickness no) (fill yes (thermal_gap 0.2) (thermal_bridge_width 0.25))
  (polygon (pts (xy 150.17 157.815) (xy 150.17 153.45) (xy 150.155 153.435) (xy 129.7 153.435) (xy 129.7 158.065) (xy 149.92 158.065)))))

